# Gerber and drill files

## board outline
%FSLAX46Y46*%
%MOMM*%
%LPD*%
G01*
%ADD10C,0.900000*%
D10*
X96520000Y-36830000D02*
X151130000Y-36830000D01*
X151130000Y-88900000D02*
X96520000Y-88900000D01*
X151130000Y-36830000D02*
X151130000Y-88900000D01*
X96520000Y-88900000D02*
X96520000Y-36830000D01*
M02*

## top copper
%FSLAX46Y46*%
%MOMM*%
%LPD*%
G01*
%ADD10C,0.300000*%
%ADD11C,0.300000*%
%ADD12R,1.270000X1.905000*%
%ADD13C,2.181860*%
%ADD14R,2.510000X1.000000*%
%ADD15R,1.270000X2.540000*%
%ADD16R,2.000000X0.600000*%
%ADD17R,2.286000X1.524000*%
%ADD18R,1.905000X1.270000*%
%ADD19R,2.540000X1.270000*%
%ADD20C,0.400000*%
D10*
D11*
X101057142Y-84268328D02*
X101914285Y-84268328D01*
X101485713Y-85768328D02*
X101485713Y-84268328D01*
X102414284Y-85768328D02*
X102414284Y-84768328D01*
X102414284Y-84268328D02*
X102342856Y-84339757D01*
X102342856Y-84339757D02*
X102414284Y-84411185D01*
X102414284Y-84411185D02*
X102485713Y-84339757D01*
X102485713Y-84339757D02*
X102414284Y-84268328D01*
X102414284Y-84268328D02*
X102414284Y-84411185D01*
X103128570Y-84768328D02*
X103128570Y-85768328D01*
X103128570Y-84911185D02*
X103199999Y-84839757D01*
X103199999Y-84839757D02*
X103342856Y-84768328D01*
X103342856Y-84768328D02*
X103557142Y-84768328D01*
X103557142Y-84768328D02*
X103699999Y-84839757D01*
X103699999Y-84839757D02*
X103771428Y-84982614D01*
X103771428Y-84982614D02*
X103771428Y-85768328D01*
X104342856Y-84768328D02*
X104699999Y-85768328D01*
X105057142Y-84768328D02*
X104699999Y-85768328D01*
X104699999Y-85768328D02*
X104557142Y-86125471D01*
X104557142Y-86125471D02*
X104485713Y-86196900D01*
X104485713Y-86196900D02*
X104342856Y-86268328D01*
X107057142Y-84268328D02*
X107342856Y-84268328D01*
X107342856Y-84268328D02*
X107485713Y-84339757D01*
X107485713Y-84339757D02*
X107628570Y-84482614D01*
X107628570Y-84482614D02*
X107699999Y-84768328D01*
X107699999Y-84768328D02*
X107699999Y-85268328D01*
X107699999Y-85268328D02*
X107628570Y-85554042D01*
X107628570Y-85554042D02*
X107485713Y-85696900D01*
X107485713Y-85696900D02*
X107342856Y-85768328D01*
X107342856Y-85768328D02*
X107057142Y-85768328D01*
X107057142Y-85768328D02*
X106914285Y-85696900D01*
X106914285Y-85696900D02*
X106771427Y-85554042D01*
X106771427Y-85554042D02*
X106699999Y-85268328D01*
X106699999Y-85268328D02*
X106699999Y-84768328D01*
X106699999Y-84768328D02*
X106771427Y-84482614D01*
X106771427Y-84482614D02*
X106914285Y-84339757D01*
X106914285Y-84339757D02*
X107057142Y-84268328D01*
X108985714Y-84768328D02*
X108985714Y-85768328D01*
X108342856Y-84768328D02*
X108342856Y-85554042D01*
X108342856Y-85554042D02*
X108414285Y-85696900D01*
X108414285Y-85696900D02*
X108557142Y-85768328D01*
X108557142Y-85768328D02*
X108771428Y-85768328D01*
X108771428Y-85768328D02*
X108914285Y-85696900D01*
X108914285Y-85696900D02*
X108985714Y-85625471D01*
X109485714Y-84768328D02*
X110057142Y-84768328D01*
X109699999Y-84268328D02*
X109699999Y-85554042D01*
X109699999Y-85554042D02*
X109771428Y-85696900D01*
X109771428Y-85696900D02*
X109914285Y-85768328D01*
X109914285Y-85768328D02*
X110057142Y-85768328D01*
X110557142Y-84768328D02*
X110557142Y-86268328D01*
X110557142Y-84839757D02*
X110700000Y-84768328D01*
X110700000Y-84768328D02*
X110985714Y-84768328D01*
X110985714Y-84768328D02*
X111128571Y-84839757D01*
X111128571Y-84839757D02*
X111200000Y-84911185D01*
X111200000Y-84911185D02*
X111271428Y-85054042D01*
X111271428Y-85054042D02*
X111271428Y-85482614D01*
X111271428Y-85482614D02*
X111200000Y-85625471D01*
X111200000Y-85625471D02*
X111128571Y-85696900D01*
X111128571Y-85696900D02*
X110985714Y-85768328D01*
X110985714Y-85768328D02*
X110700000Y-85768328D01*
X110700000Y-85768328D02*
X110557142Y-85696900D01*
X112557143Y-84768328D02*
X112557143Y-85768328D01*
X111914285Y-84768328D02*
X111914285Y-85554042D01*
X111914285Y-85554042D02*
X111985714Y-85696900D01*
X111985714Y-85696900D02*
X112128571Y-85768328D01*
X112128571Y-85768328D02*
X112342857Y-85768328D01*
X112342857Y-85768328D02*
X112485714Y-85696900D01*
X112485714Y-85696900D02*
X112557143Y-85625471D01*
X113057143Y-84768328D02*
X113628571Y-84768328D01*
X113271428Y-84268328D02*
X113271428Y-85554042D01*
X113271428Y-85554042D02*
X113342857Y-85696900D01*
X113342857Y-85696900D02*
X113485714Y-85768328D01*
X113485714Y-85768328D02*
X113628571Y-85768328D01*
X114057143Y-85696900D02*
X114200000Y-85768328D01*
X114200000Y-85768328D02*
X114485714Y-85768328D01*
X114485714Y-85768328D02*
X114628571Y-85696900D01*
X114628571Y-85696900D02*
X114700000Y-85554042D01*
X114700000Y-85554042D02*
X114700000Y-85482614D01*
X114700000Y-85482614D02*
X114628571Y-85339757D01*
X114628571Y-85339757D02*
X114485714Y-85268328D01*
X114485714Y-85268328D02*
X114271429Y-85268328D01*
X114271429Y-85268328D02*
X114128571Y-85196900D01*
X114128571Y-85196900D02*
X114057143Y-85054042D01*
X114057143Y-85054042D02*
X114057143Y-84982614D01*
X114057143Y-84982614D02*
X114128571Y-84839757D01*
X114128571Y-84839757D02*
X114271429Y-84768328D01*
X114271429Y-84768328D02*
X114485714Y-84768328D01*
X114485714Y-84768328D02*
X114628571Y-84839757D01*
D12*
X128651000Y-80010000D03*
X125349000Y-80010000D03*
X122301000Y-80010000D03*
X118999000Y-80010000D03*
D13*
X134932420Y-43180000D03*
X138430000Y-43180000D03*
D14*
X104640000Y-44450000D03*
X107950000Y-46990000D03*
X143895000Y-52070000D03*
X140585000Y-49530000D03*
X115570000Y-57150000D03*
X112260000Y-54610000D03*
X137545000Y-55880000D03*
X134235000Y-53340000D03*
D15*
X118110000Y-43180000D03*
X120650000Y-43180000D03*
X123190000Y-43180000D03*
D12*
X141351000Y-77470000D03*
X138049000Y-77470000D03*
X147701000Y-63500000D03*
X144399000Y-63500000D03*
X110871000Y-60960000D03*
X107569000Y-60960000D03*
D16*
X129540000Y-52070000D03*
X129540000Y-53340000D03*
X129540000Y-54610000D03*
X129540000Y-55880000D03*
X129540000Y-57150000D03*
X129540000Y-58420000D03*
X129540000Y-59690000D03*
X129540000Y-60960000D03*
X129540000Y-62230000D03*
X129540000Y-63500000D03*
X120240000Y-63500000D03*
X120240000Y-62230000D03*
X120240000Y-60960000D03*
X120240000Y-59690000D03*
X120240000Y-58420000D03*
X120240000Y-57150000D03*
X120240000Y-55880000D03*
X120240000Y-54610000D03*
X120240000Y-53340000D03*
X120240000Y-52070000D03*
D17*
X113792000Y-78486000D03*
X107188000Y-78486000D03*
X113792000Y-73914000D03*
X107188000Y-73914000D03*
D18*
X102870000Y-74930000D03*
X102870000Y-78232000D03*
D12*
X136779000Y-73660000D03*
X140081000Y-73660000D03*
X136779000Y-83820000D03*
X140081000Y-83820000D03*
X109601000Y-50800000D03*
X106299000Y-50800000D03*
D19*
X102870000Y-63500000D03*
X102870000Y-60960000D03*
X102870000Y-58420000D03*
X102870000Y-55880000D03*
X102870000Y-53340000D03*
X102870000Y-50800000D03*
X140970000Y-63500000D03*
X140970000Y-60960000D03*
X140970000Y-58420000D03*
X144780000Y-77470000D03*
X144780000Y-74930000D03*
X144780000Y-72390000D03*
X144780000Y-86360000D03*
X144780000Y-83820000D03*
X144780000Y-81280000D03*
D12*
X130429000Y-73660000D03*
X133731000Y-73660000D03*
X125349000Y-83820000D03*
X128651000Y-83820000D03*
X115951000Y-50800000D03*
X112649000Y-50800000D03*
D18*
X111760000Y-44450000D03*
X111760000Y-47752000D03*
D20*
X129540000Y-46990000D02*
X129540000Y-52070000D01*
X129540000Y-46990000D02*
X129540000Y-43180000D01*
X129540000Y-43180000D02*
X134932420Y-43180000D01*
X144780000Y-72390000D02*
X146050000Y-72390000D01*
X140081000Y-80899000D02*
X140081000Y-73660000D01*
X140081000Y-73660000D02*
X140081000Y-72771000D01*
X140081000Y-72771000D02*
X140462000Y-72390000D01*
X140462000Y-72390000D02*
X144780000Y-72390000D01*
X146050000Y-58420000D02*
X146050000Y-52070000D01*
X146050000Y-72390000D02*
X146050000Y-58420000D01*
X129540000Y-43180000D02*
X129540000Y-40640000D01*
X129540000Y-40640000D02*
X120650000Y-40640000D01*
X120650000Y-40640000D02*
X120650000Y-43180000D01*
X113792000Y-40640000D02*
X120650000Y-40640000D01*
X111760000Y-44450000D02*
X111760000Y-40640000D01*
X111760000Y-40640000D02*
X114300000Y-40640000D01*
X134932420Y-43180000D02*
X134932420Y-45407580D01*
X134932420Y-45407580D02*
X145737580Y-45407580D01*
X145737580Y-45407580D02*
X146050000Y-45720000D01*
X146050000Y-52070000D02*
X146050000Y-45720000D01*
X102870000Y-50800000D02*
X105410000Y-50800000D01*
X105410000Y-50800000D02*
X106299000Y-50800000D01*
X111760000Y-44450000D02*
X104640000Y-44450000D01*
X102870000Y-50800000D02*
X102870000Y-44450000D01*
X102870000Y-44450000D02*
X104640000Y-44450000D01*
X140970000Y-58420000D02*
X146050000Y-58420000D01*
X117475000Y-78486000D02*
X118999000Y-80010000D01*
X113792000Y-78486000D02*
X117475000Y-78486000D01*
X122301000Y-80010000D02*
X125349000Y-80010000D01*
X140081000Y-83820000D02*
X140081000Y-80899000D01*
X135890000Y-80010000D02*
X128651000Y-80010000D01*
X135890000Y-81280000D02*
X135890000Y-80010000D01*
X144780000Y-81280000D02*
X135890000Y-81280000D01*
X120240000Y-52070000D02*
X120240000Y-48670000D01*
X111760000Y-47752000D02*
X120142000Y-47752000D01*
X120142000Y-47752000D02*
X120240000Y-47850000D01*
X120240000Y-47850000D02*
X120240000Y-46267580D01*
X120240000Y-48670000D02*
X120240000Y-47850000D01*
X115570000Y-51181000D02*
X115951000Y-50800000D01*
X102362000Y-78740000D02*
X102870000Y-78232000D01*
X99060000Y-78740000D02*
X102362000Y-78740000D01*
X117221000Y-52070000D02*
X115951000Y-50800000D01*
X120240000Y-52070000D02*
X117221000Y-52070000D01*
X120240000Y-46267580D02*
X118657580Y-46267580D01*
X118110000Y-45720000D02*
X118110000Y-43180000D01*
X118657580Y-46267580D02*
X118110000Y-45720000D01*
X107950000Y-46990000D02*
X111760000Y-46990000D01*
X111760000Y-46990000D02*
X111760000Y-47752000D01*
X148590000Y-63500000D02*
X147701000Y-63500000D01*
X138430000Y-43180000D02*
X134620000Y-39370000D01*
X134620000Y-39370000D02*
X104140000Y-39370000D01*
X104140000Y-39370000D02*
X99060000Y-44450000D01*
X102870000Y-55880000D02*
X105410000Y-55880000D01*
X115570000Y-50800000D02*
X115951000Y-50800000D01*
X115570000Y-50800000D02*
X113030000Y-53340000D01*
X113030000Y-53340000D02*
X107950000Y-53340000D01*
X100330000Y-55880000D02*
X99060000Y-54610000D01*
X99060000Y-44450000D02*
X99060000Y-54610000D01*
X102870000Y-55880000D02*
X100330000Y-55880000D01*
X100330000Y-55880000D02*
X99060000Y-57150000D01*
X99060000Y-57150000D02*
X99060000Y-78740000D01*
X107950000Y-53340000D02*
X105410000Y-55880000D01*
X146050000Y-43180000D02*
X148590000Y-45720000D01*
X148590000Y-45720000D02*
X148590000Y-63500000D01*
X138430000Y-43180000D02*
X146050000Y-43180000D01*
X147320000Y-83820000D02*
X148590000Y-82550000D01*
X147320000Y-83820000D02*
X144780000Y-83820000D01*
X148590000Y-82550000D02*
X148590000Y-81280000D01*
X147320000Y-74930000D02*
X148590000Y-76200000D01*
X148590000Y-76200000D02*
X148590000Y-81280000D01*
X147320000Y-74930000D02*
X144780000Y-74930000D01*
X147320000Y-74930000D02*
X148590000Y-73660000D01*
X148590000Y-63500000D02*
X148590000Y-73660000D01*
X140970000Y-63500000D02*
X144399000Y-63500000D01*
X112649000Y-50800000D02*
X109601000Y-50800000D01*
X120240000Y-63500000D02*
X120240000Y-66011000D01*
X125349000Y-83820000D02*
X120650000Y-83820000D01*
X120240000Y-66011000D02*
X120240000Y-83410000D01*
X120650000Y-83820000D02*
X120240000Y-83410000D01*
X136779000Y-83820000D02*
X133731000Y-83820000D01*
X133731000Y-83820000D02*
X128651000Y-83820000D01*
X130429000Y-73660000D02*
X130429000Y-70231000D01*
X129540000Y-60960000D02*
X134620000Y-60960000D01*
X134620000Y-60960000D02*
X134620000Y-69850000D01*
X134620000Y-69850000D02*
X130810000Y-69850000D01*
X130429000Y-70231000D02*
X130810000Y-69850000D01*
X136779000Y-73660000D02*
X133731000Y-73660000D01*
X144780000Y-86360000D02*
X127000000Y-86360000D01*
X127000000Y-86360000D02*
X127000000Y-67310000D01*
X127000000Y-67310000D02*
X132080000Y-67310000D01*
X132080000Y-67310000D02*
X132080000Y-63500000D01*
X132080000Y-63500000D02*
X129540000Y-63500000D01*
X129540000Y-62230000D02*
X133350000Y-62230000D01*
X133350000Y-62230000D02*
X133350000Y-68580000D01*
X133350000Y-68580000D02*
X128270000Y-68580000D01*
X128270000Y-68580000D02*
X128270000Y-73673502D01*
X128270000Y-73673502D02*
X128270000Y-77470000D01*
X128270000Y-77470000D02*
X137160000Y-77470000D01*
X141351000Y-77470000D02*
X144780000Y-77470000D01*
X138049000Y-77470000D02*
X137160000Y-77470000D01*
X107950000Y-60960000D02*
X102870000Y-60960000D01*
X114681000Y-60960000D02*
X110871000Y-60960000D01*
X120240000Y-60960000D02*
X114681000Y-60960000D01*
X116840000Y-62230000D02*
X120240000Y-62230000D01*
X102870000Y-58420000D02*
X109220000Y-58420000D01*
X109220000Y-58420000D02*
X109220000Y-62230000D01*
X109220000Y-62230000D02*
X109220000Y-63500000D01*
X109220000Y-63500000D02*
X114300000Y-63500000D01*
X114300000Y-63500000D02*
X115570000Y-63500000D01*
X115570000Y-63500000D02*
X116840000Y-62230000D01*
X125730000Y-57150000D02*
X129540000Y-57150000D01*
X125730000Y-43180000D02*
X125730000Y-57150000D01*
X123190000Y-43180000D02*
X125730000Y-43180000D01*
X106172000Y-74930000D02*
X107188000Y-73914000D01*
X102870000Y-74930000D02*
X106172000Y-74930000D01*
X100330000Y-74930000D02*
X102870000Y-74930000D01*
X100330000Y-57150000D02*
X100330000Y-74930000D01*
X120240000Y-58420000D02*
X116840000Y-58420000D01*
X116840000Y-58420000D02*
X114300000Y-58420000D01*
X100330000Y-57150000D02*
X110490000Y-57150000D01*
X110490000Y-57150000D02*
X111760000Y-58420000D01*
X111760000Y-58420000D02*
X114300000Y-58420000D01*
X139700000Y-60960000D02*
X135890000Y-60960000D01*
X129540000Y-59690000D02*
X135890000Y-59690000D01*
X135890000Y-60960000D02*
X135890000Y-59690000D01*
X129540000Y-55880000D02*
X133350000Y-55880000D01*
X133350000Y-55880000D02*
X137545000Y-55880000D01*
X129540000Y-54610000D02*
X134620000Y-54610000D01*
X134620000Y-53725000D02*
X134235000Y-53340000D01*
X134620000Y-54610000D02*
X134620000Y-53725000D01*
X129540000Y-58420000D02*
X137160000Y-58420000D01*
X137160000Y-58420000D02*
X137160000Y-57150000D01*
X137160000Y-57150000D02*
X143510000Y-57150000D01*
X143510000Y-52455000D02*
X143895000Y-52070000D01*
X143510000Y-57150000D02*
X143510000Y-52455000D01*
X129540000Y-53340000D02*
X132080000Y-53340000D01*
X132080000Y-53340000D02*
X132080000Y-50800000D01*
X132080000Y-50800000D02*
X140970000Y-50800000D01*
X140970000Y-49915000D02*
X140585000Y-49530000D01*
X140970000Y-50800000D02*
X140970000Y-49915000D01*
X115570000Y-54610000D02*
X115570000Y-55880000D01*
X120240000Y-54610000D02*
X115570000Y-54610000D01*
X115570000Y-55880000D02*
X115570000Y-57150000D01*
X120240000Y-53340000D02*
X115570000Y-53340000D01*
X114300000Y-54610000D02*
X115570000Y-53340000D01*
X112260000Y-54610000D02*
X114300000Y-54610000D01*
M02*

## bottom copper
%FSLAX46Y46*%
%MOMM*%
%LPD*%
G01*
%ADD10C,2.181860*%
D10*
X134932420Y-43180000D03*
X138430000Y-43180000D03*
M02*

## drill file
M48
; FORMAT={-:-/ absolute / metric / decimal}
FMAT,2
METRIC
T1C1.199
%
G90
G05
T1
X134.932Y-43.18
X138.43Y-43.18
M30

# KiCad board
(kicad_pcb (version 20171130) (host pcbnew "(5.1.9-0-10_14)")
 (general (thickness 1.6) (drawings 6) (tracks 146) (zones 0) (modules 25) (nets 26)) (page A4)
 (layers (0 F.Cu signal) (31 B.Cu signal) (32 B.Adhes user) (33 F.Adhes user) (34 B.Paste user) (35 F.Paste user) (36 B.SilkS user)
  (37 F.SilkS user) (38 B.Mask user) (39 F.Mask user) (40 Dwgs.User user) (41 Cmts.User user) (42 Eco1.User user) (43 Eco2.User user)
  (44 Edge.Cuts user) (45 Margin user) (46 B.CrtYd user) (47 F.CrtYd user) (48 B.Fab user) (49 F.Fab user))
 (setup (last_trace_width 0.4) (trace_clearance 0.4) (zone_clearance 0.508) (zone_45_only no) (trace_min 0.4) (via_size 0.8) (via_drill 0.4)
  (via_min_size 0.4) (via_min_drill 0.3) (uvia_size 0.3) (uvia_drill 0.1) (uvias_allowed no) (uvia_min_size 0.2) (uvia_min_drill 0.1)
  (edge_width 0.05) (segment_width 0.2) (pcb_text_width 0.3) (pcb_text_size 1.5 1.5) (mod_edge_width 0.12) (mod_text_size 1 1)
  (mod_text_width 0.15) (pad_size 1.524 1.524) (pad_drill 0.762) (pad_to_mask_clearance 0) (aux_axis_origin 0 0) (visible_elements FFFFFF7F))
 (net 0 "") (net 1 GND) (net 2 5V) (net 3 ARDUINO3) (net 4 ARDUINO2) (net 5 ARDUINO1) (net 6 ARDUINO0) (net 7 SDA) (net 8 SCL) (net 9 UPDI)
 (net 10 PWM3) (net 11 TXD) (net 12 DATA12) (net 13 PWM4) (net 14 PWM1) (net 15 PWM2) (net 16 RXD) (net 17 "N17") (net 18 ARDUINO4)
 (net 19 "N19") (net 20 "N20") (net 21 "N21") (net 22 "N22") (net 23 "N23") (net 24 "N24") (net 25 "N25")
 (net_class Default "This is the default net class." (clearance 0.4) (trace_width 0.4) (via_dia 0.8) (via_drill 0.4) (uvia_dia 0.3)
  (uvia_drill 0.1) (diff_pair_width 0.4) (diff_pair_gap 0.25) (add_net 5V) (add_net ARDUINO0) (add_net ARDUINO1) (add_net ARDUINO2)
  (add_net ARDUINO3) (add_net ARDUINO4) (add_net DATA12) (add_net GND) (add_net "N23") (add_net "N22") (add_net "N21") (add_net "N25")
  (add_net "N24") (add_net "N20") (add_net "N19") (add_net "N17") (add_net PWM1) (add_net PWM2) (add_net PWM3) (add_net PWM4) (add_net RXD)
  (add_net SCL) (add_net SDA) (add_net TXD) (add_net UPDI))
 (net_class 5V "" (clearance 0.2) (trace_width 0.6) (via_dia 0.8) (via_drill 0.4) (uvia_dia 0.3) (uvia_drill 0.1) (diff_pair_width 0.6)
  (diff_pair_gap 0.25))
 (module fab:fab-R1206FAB (layer F.Cu) (at 127 80.01)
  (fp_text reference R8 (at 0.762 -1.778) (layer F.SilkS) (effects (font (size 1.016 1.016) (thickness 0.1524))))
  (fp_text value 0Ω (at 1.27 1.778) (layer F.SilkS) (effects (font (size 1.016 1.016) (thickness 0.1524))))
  (pad 2 smd rect (at 1.651 0) (size 1.27 1.905) (layers F.Cu F.Paste F.Mask) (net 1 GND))
  (pad 1 smd rect (at -1.651 0) (size 1.27 1.905) (layers F.Cu F.Paste F.Mask) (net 1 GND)))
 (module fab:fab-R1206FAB (layer F.Cu) (at 120.65 80.01)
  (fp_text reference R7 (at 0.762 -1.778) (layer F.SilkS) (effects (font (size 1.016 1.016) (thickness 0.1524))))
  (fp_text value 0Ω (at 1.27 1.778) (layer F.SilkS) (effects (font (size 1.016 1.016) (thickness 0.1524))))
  (pad 2 smd rect (at 1.651 0) (size 1.27 1.905) (layers F.Cu F.Paste F.Mask) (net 1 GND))
  (pad 1 smd rect (at -1.651 0) (size 1.27 1.905) (layers F.Cu F.Paste F.Mask) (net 1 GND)))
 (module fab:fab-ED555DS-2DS (layer F.Cu) (at 136.63168 43.18)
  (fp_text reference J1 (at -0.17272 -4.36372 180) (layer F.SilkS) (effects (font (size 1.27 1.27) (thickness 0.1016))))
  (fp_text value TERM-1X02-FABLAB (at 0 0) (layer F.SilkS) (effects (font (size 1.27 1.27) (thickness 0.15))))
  (pad 2 thru_hole circle (at -1.69926 0) (size 2.18186 2.18186) (drill 1.19888) (layers F&B.Cu F.Paste F.SilkS F.Mask) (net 1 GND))
  (pad 1 thru_hole circle (at 1.79832 0) (size 2.18186 2.18186) (drill 1.19888) (layers F&B.Cu F.Paste F.SilkS F.Mask) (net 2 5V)))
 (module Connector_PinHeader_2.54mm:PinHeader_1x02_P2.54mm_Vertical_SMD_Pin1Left (layer F.Cu) (at 106.295 45.72 180)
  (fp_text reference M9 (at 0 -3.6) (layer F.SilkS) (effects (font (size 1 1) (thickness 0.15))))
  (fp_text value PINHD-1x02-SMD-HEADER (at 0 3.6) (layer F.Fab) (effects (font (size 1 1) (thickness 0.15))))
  (pad 2 smd rect (at 1.655 1.27 180) (size 2.51 1) (layers F.Cu F.Paste F.Mask) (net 1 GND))
  (pad 1 smd rect (at -1.655 -1.27 180) (size 2.51 1) (layers F.Cu F.Paste F.Mask) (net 2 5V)))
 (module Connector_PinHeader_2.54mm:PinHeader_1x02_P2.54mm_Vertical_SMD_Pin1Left (layer F.Cu) (at 142.24 50.8)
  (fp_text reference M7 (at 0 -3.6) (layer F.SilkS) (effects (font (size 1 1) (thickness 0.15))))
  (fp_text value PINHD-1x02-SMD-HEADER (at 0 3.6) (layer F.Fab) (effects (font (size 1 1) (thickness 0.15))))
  (pad 2 smd rect (at 1.655 1.27) (size 2.51 1) (layers F.Cu F.Paste F.Mask) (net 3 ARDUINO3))
  (pad 1 smd rect (at -1.655 -1.27) (size 2.51 1) (layers F.Cu F.Paste F.Mask) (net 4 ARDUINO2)))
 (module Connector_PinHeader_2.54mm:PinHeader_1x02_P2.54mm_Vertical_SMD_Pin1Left (layer F.Cu) (at 113.915 55.88)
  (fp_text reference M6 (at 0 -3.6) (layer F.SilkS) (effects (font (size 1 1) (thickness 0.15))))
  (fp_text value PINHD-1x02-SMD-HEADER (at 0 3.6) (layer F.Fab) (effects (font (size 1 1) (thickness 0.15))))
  (pad 2 smd rect (at 1.655 1.27) (size 2.51 1) (layers F.Cu F.Paste F.Mask) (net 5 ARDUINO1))
  (pad 1 smd rect (at -1.655 -1.27) (size 2.51 1) (layers F.Cu F.Paste F.Mask) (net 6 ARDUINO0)))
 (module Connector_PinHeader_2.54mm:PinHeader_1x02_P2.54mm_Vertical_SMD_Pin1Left (layer F.Cu) (at 135.89 54.61)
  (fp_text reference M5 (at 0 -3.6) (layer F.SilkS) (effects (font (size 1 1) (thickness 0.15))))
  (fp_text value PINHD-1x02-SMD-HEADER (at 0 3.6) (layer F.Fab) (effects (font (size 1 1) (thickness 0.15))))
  (pad 2 smd rect (at 1.655 1.27) (size 2.51 1) (layers F.Cu F.Paste F.Mask) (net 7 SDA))
  (pad 1 smd rect (at -1.655 -1.27) (size 2.51 1) (layers F.Cu F.Paste F.Mask) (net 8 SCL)))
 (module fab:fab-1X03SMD (layer F.Cu) (at 120.65 43.18 270)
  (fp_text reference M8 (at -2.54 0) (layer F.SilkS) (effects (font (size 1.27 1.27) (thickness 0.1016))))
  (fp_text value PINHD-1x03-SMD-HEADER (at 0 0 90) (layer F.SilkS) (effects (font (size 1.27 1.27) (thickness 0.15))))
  (pad 3 smd rect (at 0 2.54 270) (size 2.54 1.27) (layers F.Cu F.Paste F.Mask) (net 2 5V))
  (pad 2 smd rect (at 0 0 270) (size 2.54 1.27) (layers F.Cu F.Paste F.Mask) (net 1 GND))
  (pad 1 smd rect (at 0 -2.54 270) (size 2.54 1.27) (layers F.Cu F.Paste F.Mask) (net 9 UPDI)))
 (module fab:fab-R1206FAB (layer F.Cu) (at 139.7 77.47)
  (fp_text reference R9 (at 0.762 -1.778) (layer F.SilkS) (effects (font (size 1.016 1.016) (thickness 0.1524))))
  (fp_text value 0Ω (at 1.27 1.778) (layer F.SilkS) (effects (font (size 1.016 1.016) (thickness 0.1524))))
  (pad 2 smd rect (at 1.651 0) (size 1.27 1.905) (layers F.Cu F.Paste F.Mask) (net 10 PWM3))
  (pad 1 smd rect (at -1.651 0) (size 1.27 1.905) (layers F.Cu F.Paste F.Mask) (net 10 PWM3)))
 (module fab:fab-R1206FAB (layer F.Cu) (at 146.05 63.5)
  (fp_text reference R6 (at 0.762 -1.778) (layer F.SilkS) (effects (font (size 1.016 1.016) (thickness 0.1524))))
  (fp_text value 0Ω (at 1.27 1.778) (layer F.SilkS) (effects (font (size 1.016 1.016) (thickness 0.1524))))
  (pad 2 smd rect (at 1.651 0) (size 1.27 1.905) (layers F.Cu F.Paste F.Mask) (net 2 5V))
  (pad 1 smd rect (at -1.651 0) (size 1.27 1.905) (layers F.Cu F.Paste F.Mask) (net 2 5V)))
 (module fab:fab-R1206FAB (layer F.Cu) (at 109.22 60.96)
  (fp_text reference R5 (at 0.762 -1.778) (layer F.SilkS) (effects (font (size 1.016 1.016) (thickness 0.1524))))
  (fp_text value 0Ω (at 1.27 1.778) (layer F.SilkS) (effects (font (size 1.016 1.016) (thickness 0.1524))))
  (pad 2 smd rect (at 1.651 0) (size 1.27 1.905) (layers F.Cu F.Paste F.Mask) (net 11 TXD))
  (pad 1 smd rect (at -1.651 0) (size 1.27 1.905) (layers F.Cu F.Paste F.Mask) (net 11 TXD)))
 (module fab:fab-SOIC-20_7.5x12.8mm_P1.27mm (layer F.Cu) (at 124.89 57.785)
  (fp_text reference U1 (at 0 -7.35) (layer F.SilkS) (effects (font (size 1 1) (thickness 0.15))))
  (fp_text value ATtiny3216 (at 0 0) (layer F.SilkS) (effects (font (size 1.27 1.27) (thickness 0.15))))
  (pad 20 smd rect (at 4.65 -5.715) (size 2 0.6) (layers F.Cu) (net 1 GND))
  (pad 19 smd rect (at 4.65 -4.445) (size 2 0.6) (layers F.Cu) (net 4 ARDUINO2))
  (pad 18 smd rect (at 4.65 -3.175) (size 2 0.6) (layers F.Cu) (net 8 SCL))
  (pad 17 smd rect (at 4.65 -1.905) (size 2 0.6) (layers F.Cu) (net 7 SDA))
  (pad 16 smd rect (at 4.65 -0.635) (size 2 0.6) (layers F.Cu) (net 9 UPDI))
  (pad 15 smd rect (at 4.65 0.635) (size 2 0.6) (layers F.Cu) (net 3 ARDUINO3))
  (pad 14 smd rect (at 4.65 1.905) (size 2 0.6) (layers F.Cu) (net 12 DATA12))
  (pad 13 smd rect (at 4.65 3.175) (size 2 0.6) (layers F.Cu) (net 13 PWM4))
  (pad 12 smd rect (at 4.65 4.445) (size 2 0.6) (layers F.Cu) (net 10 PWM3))
  (pad 11 smd rect (at 4.65 5.715) (size 2 0.6) (layers F.Cu) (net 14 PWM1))
  (pad 10 smd rect (at -4.65 5.715) (size 2 0.6) (layers F.Cu) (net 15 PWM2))
  (pad 9 smd rect (at -4.65 4.445) (size 2 0.6) (layers F.Cu) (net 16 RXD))
  (pad 8 smd rect (at -4.65 3.175) (size 2 0.6) (layers F.Cu) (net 11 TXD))
  (pad 7 smd rect (at -4.65 1.905) (size 2 0.6) (layers F.Cu) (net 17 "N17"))
  (pad 6 smd rect (at -4.65 0.635) (size 2 0.6) (layers F.Cu) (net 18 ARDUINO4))
  (pad 5 smd rect (at -4.65 -0.635) (size 2 0.6) (layers F.Cu) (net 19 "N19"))
  (pad 4 smd rect (at -4.65 -1.905) (size 2 0.6) (layers F.Cu) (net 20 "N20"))
  (pad 3 smd rect (at -4.65 -3.175) (size 2 0.6) (layers F.Cu) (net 5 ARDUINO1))
  (pad 2 smd rect (at -4.65 -4.445) (size 2 0.6) (layers F.Cu) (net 6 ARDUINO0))
  (pad 1 smd rect (at -4.65 -5.715) (size 2 0.6) (layers F.Cu) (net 2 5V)))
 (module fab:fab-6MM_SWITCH (layer F.Cu) (at 110.49 76.2)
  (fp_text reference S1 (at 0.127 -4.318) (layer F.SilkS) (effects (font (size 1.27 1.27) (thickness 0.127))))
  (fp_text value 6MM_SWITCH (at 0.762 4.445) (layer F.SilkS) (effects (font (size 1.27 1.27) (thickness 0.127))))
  (pad 4 smd rect (at 3.302 2.286) (size 2.286 1.524) (layers F.Cu F.Paste F.Mask) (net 1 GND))
  (pad 3 smd rect (at -3.302 2.286) (size 2.286 1.524) (layers F.Cu F.Paste F.Mask) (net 1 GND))
  (pad 2 smd rect (at 3.302 -2.286) (size 2.286 1.524) (layers F.Cu F.Paste F.Mask) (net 18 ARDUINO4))
  (pad 1 smd rect (at -3.302 -2.286) (size 2.286 1.524) (layers F.Cu F.Paste F.Mask) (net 18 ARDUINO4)))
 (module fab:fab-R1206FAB (layer F.Cu) (at 102.87 76.581 90)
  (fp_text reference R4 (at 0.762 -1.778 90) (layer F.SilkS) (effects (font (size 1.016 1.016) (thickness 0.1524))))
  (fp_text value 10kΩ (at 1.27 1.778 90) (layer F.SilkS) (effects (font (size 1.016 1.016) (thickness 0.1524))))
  (pad 2 smd rect (at 1.651 0 90) (size 1.27 1.905) (layers F.Cu F.Paste F.Mask) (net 18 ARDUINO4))
  (pad 1 smd rect (at -1.651 0 90) (size 1.27 1.905) (layers F.Cu F.Paste F.Mask) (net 2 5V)))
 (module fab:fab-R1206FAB (layer F.Cu) (at 138.43 73.66 180)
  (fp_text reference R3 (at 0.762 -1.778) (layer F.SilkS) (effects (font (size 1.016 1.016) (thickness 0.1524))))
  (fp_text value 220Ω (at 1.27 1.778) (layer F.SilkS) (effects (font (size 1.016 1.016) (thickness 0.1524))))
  (pad 2 smd rect (at 1.651 0 180) (size 1.27 1.905) (layers F.Cu F.Paste F.Mask) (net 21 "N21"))
  (pad 1 smd rect (at -1.651 0 180) (size 1.27 1.905) (layers F.Cu F.Paste F.Mask) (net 1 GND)))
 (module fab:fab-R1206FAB (layer F.Cu) (at 138.43 83.82 180)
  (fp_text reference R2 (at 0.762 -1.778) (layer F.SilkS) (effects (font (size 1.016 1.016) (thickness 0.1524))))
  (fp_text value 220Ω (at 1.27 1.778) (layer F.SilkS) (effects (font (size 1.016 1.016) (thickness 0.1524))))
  (pad 2 smd rect (at 1.651 0 180) (size 1.27 1.905) (layers F.Cu F.Paste F.Mask) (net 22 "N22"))
  (pad 1 smd rect (at -1.651 0 180) (size 1.27 1.905) (layers F.Cu F.Paste F.Mask) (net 1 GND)))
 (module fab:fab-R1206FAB (layer F.Cu) (at 107.95 50.8)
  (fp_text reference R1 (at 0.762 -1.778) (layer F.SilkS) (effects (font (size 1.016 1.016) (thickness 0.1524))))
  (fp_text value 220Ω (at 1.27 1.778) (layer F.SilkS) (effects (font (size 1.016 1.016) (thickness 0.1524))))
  (pad 2 smd rect (at 1.651 0) (size 1.27 1.905) (layers F.Cu F.Paste F.Mask) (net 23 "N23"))
  (pad 1 smd rect (at -1.651 0) (size 1.27 1.905) (layers F.Cu F.Paste F.Mask) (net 1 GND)))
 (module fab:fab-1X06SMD (layer F.Cu) (at 102.87 57.15)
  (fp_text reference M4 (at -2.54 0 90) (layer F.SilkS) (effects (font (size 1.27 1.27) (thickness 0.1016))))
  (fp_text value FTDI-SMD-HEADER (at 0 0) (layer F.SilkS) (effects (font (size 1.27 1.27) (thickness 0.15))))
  (pad 6 smd rect (at 0 6.35) (size 2.54 1.27) (layers F.Cu F.Paste F.Mask) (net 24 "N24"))
  (pad 5 smd rect (at 0 3.81) (size 2.54 1.27) (layers F.Cu F.Paste F.Mask) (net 11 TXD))
  (pad 4 smd rect (at 0 1.27) (size 2.54 1.27) (layers F.Cu F.Paste F.Mask) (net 16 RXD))
  (pad 3 smd rect (at 0 -1.27) (size 2.54 1.27) (layers F.Cu F.Paste F.Mask) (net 2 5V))
  (pad 2 smd rect (at 0 -3.81) (size 2.54 1.27) (layers F.Cu F.Paste F.Mask) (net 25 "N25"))
  (pad 1 smd rect (at 0 -6.35) (size 2.54 1.27) (layers F.Cu F.Paste F.Mask) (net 1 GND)))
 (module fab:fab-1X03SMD (layer F.Cu) (at 140.97 60.96)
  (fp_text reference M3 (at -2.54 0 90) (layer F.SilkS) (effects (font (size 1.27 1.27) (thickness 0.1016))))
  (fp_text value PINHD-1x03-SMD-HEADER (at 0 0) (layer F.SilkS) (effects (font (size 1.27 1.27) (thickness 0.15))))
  (pad 3 smd rect (at 0 2.54) (size 2.54 1.27) (layers F.Cu F.Paste F.Mask) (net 2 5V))
  (pad 2 smd rect (at 0 0) (size 2.54 1.27) (layers F.Cu F.Paste F.Mask) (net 12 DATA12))
  (pad 1 smd rect (at 0 -2.54) (size 2.54 1.27) (layers F.Cu F.Paste F.Mask) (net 1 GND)))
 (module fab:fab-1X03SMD (layer F.Cu) (at 144.78 74.93)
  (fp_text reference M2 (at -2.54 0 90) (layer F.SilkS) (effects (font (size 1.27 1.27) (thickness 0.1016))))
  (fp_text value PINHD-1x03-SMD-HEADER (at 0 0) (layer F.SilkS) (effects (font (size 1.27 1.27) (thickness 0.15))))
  (pad 3 smd rect (at 0 2.54) (size 2.54 1.27) (layers F.Cu F.Paste F.Mask) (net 10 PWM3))
  (pad 2 smd rect (at 0 0) (size 2.54 1.27) (layers F.Cu F.Paste F.Mask) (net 2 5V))
  (pad 1 smd rect (at 0 -2.54) (size 2.54 1.27) (layers F.Cu F.Paste F.Mask) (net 1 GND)))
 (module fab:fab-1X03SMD (layer F.Cu) (at 144.78 83.82)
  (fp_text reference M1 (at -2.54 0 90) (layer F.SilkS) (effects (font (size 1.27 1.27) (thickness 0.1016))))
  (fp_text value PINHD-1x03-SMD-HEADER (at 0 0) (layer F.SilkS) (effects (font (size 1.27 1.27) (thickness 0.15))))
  (pad 3 smd rect (at 0 2.54) (size 2.54 1.27) (layers F.Cu F.Paste F.Mask) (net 14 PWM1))
  (pad 2 smd rect (at 0 0) (size 2.54 1.27) (layers F.Cu F.Paste F.Mask) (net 2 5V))
  (pad 1 smd rect (at 0 -2.54) (size 2.54 1.27) (layers F.Cu F.Paste F.Mask) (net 1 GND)))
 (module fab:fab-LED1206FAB (layer F.Cu) (at 132.08 73.66 180)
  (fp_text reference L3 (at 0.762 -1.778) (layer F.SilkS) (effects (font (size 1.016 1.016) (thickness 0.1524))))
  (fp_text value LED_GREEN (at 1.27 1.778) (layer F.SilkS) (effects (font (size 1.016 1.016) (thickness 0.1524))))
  (pad 2 smd rect (at 1.651 0 180) (size 1.27 1.905) (layers F.Cu F.Paste F.Mask) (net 13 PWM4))
  (pad 1 smd rect (at -1.651 0 180) (size 1.27 1.905) (layers F.Cu F.Paste F.Mask) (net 21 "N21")))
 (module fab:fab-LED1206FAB (layer F.Cu) (at 127 83.82 180)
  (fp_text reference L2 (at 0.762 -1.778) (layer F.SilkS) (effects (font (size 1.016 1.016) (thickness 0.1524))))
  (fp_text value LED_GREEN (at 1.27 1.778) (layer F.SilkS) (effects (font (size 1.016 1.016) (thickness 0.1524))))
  (pad 2 smd rect (at 1.651 0 180) (size 1.27 1.905) (layers F.Cu F.Paste F.Mask) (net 15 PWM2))
  (pad 1 smd rect (at -1.651 0 180) (size 1.27 1.905) (layers F.Cu F.Paste F.Mask) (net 22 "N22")))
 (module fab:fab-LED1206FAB (layer F.Cu) (at 114.3 50.8)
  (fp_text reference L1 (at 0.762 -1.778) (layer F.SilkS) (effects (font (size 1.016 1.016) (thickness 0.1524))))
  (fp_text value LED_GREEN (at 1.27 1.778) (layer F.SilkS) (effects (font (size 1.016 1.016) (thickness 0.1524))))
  (pad 2 smd rect (at 1.651 0) (size 1.27 1.905) (layers F.Cu F.Paste F.Mask) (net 2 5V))
  (pad 1 smd rect (at -1.651 0) (size 1.27 1.905) (layers F.Cu F.Paste F.Mask) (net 23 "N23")))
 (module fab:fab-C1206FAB (layer F.Cu) (at 111.76 46.101 90)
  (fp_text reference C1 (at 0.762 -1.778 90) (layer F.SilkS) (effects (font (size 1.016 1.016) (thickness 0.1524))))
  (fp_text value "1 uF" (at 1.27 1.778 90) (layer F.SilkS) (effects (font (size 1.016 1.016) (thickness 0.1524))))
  (pad 2 smd rect (at 1.651 0 90) (size 1.27 1.905) (layers F.Cu F.Paste F.Mask) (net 1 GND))
  (pad 1 smd rect (at -1.651 0 90) (size 1.27 1.905) (layers F.Cu F.Paste F.Mask) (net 2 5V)))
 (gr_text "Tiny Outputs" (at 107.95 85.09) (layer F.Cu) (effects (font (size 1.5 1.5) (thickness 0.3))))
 (gr_line (start 96.52 36.83) (end 151.13 36.83) (layer Edge.Cuts) (width 0.9))
 (gr_line (start 151.13 88.9) (end 96.52 88.9) (layer Edge.Cuts) (width 0.9))
 (gr_line (start 151.13 36.83) (end 151.13 88.9) (layer Edge.Cuts) (width 0.9))
 (gr_line (start 96.52 88.9) (end 96.52 36.83) (layer Edge.Cuts) (width 0.9))
 (segment (start 129.54 46.99) (end 129.54 52.07) (width 0.4) (layer F.Cu) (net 1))
 (segment (start 129.54 46.99) (end 129.54 43.18) (width 0.4) (layer F.Cu) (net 1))
 (segment (start 129.54 43.18) (end 134.93242 43.18) (width 0.4) (layer F.Cu) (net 1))
 (segment (start 144.78 72.39) (end 146.05 72.39) (width 0.4) (layer F.Cu) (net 1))
 (segment (start 140.081 80.899) (end 140.081 73.66) (width 0.4) (layer F.Cu) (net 1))
 (segment (start 140.081 73.66) (end 140.081 72.771) (width 0.4) (layer F.Cu) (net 1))
 (segment (start 140.081 72.771) (end 140.462 72.39) (width 0.4) (layer F.Cu) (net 1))
 (segment (start 140.462 72.39) (end 144.78 72.39) (width 0.4) (layer F.Cu) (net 1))
 (segment (start 146.05 58.42) (end 146.05 52.07) (width 0.4) (layer F.Cu) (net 1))
 (segment (start 146.05 72.39) (end 146.05 58.42) (width 0.4) (layer F.Cu) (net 1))
 (segment (start 129.54 43.18) (end 129.54 40.64) (width 0.4) (layer F.Cu) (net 1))
 (segment (start 129.54 40.64) (end 120.65 40.64) (width 0.4) (layer F.Cu) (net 1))
 (segment (start 120.65 40.64) (end 120.65 43.18) (width 0.4) (layer F.Cu) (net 1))
 (segment (start 113.792 40.64) (end 120.65 40.64) (width 0.4) (layer F.Cu) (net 1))
 (segment (start 111.76 44.45) (end 111.76 40.64) (width 0.4) (layer F.Cu) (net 1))
 (segment (start 111.76 40.64) (end 114.3 40.64) (width 0.4) (layer F.Cu) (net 1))
 (segment (start 134.93242 43.18) (end 134.93242 45.40758) (width 0.4) (layer F.Cu) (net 1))
 (segment (start 134.93242 45.40758) (end 145.73758 45.40758) (width 0.4) (layer F.Cu) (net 1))
 (segment (start 145.73758 45.40758) (end 146.05 45.72) (width 0.4) (layer F.Cu) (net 1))
 (segment (start 146.05 52.07) (end 146.05 45.72) (width 0.4) (layer F.Cu) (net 1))
 (segment (start 102.87 50.8) (end 105.41 50.8) (width 0.4) (layer F.Cu) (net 1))
 (segment (start 105.41 50.8) (end 106.299 50.8) (width 0.4) (layer F.Cu) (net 1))
 (segment (start 111.76 44.45) (end 104.64 44.45) (width 0.4) (layer F.Cu) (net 1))
 (segment (start 102.87 50.8) (end 102.87 44.45) (width 0.4) (layer F.Cu) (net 1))
 (segment (start 102.87 44.45) (end 104.64 44.45) (width 0.4) (layer F.Cu) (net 1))
 (segment (start 140.97 58.42) (end 146.05 58.42) (width 0.4) (layer F.Cu) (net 1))
 (segment (start 117.475 78.486) (end 118.999 80.01) (width 0.4) (layer F.Cu) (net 1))
 (segment (start 113.792 78.486) (end 117.475 78.486) (width 0.4) (layer F.Cu) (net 1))
 (segment (start 122.301 80.01) (end 125.349 80.01) (width 0.4) (layer F.Cu) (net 1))
 (segment (start 140.081 83.82) (end 140.081 80.899) (width 0.4) (layer F.Cu) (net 1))
 (segment (start 135.89 80.01) (end 128.651 80.01) (width 0.4) (layer F.Cu) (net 1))
 (segment (start 135.89 81.28) (end 135.89 80.01) (width 0.4) (layer F.Cu) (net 1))
 (segment (start 144.78 81.28) (end 135.89 81.28) (width 0.4) (layer F.Cu) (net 1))
 (segment (start 120.24 52.07) (end 120.24 48.67) (width 0.4) (layer F.Cu) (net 2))
 (segment (start 111.76 47.752) (end 120.142 47.752) (width 0.4) (layer F.Cu) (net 2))
 (segment (start 120.142 47.752) (end 120.24 47.85) (width 0.4) (layer F.Cu) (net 2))
 (segment (start 120.24 47.85) (end 120.24 46.26758) (width 0.4) (layer F.Cu) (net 2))
 (segment (start 120.24 48.67) (end 120.24 47.85) (width 0.4) (layer F.Cu) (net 2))
 (segment (start 115.57 51.181) (end 115.951 50.8) (width 0.4) (layer F.Cu) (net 2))
 (segment (start 102.362 78.74) (end 102.87 78.232) (width 0.4) (layer F.Cu) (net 2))
 (segment (start 99.06 78.74) (end 102.362 78.74) (width 0.4) (layer F.Cu) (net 2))
 (segment (start 117.221 52.07) (end 115.951 50.8) (width 0.4) (layer F.Cu) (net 2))
 (segment (start 120.24 52.07) (end 117.221 52.07) (width 0.4) (layer F.Cu) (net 2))
 (segment (start 120.24 46.26758) (end 118.65758 46.26758) (width 0.4) (layer F.Cu) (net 2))
 (segment (start 118.11 45.72) (end 118.11 43.18) (width 0.4) (layer F.Cu) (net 2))
 (segment (start 118.65758 46.26758) (end 118.11 45.72) (width 0.4) (layer F.Cu) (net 2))
 (segment (start 107.95 46.99) (end 111.76 46.99) (width 0.4) (layer F.Cu) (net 2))
 (segment (start 111.76 46.99) (end 111.76 47.752) (width 0.4) (layer F.Cu) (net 2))
 (segment (start 148.59 63.5) (end 147.701 63.5) (width 0.4) (layer F.Cu) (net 2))
 (segment (start 138.43 43.18) (end 134.62 39.37) (width 0.4) (layer F.Cu) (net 2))
 (segment (start 134.62 39.37) (end 104.14 39.37) (width 0.4) (layer F.Cu) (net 2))
 (segment (start 104.14 39.37) (end 99.06 44.45) (width 0.4) (layer F.Cu) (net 2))
 (segment (start 102.87 55.88) (end 105.41 55.88) (width 0.4) (layer F.Cu) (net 2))
 (segment (start 115.57 50.8) (end 115.951 50.8) (width 0.4) (layer F.Cu) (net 2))
 (segment (start 115.57 50.8) (end 113.03 53.34) (width 0.4) (layer F.Cu) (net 2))
 (segment (start 113.03 53.34) (end 107.95 53.34) (width 0.4) (layer F.Cu) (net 2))
 (segment (start 100.33 55.88) (end 99.06 54.61) (width 0.4) (layer F.Cu) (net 2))
 (segment (start 99.06 44.45) (end 99.06 54.61) (width 0.4) (layer F.Cu) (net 2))
 (segment (start 102.87 55.88) (end 100.33 55.88) (width 0.4) (layer F.Cu) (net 2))
 (segment (start 100.33 55.88) (end 99.06 57.15) (width 0.4) (layer F.Cu) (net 2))
 (segment (start 99.06 57.15) (end 99.06 78.74) (width 0.4) (layer F.Cu) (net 2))
 (segment (start 107.95 53.34) (end 105.41 55.88) (width 0.4) (layer F.Cu) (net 2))
 (segment (start 146.05 43.18) (end 148.59 45.72) (width 0.4) (layer F.Cu) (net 2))
 (segment (start 148.59 45.72) (end 148.59 63.5) (width 0.4) (layer F.Cu) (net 2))
 (segment (start 138.43 43.18) (end 146.05 43.18) (width 0.4) (layer F.Cu) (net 2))
 (segment (start 147.32 83.82) (end 148.59 82.55) (width 0.4) (layer F.Cu) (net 2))
 (segment (start 147.32 83.82) (end 144.78 83.82) (width 0.4) (layer F.Cu) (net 2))
 (segment (start 148.59 82.55) (end 148.59 81.28) (width 0.4) (layer F.Cu) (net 2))
 (segment (start 147.32 74.93) (end 148.59 76.2) (width 0.4) (layer F.Cu) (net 2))
 (segment (start 148.59 76.2) (end 148.59 81.28) (width 0.4) (layer F.Cu) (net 2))
 (segment (start 147.32 74.93) (end 144.78 74.93) (width 0.4) (layer F.Cu) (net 2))
 (segment (start 147.32 74.93) (end 148.59 73.66) (width 0.4) (layer F.Cu) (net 2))
 (segment (start 148.59 63.5) (end 148.59 73.66) (width 0.4) (layer F.Cu) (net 2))
 (segment (start 140.97 63.5) (end 144.399 63.5) (width 0.4) (layer F.Cu) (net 2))
 (segment (start 112.649 50.8) (end 109.601 50.8) (width 0.4) (layer F.Cu) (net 23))
 (segment (start 120.24 63.5) (end 120.24 66.011) (width 0.4) (layer F.Cu) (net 15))
 (segment (start 125.349 83.82) (end 120.65 83.82) (width 0.4) (layer F.Cu) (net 15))
 (segment (start 120.24 66.011) (end 120.24 83.41) (width 0.4) (layer F.Cu) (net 15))
 (segment (start 120.65 83.82) (end 120.24 83.41) (width 0.4) (layer F.Cu) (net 15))
 (segment (start 136.779 83.82) (end 133.731 83.82) (width 0.4) (layer F.Cu) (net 22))
 (segment (start 133.731 83.82) (end 128.651 83.82) (width 0.4) (layer F.Cu) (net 22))
 (segment (start 130.429 73.66) (end 130.429 70.231) (width 0.4) (layer F.Cu) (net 13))
 (segment (start 129.54 60.96) (end 134.62 60.96) (width 0.4) (layer F.Cu) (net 13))
 (segment (start 134.62 60.96) (end 134.62 69.85) (width 0.4) (layer F.Cu) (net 13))
 (segment (start 134.62 69.85) (end 130.81 69.85) (width 0.4) (layer F.Cu) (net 13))
 (segment (start 130.429 70.231) (end 130.81 69.85) (width 0.4) (layer F.Cu) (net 13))
 (segment (start 136.779 73.66) (end 133.731 73.66) (width 0.4) (layer F.Cu) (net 21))
 (segment (start 144.78 86.36) (end 127 86.36) (width 0.4) (layer F.Cu) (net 14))
 (segment (start 127 86.36) (end 127 67.31) (width 0.4) (layer F.Cu) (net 14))
 (segment (start 127 67.31) (end 132.08 67.31) (width 0.4) (layer F.Cu) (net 14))
 (segment (start 132.08 67.31) (end 132.08 63.5) (width 0.4) (layer F.Cu) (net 14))
 (segment (start 132.08 63.5) (end 129.54 63.5) (width 0.4) (layer F.Cu) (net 14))
 (segment (start 129.54 62.23) (end 133.35 62.23) (width 0.4) (layer F.Cu) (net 10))
 (segment (start 133.35 62.23) (end 133.35 68.58) (width 0.4) (layer F.Cu) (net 10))
 (segment (start 133.35 68.58) (end 128.27 68.58) (width 0.4) (layer F.Cu) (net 10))
 (segment (start 128.27 68.58) (end 128.27 73.673502) (width 0.4) (layer F.Cu) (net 10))
 (segment (start 128.27 73.673502) (end 128.27 77.47) (width 0.4) (layer F.Cu) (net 10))
 (segment (start 128.27 77.47) (end 137.16 77.47) (width 0.4) (layer F.Cu) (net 10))
 (segment (start 141.351 77.47) (end 144.78 77.47) (width 0.4) (layer F.Cu) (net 10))
 (segment (start 138.049 77.47) (end 137.16 77.47) (width 0.4) (layer F.Cu) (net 10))
 (segment (start 107.95 60.96) (end 102.87 60.96) (width 0.4) (layer F.Cu) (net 11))
 (segment (start 114.681 60.96) (end 110.871 60.96) (width 0.4) (layer F.Cu) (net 11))
 (segment (start 120.24 60.96) (end 114.681 60.96) (width 0.4) (layer F.Cu) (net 11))
 (segment (start 116.84 62.23) (end 120.24 62.23) (width 0.4) (layer F.Cu) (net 16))
 (segment (start 102.87 58.42) (end 109.22 58.42) (width 0.4) (layer F.Cu) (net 16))
 (segment (start 109.22 58.42) (end 109.22 62.23) (width 0.4) (layer F.Cu) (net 16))
 (segment (start 109.22 62.23) (end 109.22 63.5) (width 0.4) (layer F.Cu) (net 16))
 (segment (start 109.22 63.5) (end 114.3 63.5) (width 0.4) (layer F.Cu) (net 16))
 (segment (start 114.3 63.5) (end 115.57 63.5) (width 0.4) (layer F.Cu) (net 16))
 (segment (start 115.57 63.5) (end 116.84 62.23) (width 0.4) (layer F.Cu) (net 16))
 (segment (start 125.73 57.15) (end 129.54 57.15) (width 0.4) (layer F.Cu) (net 9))
 (segment (start 125.73 43.18) (end 125.73 57.15) (width 0.4) (layer F.Cu) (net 9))
 (segment (start 123.19 43.18) (end 125.73 43.18) (width 0.4) (layer F.Cu) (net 9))
 (segment (start 106.172 74.93) (end 107.188 73.914) (width 0.4) (layer F.Cu) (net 18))
 (segment (start 102.87 74.93) (end 106.172 74.93) (width 0.4) (layer F.Cu) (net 18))
 (segment (start 100.33 74.93) (end 102.87 74.93) (width 0.4) (layer F.Cu) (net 18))
 (segment (start 100.33 57.15) (end 100.33 74.93) (width 0.4) (layer F.Cu) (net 18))
 (segment (start 120.24 58.42) (end 116.84 58.42) (width 0.4) (layer F.Cu) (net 18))
 (segment (start 116.84 58.42) (end 114.3 58.42) (width 0.4) (layer F.Cu) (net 18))
 (segment (start 100.33 57.15) (end 110.49 57.15) (width 0.4) (layer F.Cu) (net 18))
 (segment (start 110.49 57.15) (end 111.76 58.42) (width 0.4) (layer F.Cu) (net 18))
 (segment (start 111.76 58.42) (end 114.3 58.42) (width 0.4) (layer F.Cu) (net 18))
 (segment (start 139.7 60.96) (end 135.89 60.96) (width 0.4) (layer F.Cu) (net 12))
 (segment (start 129.54 59.69) (end 135.89 59.69) (width 0.4) (layer F.Cu) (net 12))
 (segment (start 135.89 60.96) (end 135.89 59.69) (width 0.4) (layer F.Cu) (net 12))
 (segment (start 129.54 55.88) (end 133.35 55.88) (width 0.4) (layer F.Cu) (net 7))
 (segment (start 133.35 55.88) (end 137.545 55.88) (width 0.4) (layer F.Cu) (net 7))
 (segment (start 129.54 54.61) (end 134.62 54.61) (width 0.4) (layer F.Cu) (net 8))
 (segment (start 134.62 53.725) (end 134.235 53.34) (width 0.4) (layer F.Cu) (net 8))
 (segment (start 134.62 54.61) (end 134.62 53.725) (width 0.4) (layer F.Cu) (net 8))
 (segment (start 129.54 58.42) (end 137.16 58.42) (width 0.4) (layer F.Cu) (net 3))
 (segment (start 137.16 58.42) (end 137.16 57.15) (width 0.4) (layer F.Cu) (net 3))
 (segment (start 137.16 57.15) (end 143.51 57.15) (width 0.4) (layer F.Cu) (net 3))
 (segment (start 143.51 52.455) (end 143.895 52.07) (width 0.4) (layer F.Cu) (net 3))
 (segment (start 143.51 57.15) (end 143.51 52.455) (width 0.4) (layer F.Cu) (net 3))
 (segment (start 129.54 53.34) (end 132.08 53.34) (width 0.4) (layer F.Cu) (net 4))
 (segment (start 132.08 53.34) (end 132.08 50.8) (width 0.4) (layer F.Cu) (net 4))
 (segment (start 132.08 50.8) (end 140.97 50.8) (width 0.4) (layer F.Cu) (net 4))
 (segment (start 140.97 49.915) (end 140.585 49.53) (width 0.4) (layer F.Cu) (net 4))
 (segment (start 140.97 50.8) (end 140.97 49.915) (width 0.4) (layer F.Cu) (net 4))
 (segment (start 115.57 54.61) (end 115.57 55.88) (width 0.4) (layer F.Cu) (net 5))
 (segment (start 120.24 54.61) (end 115.57 54.61) (width 0.4) (layer F.Cu) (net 5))
 (segment (start 115.57 55.88) (end 115.57 57.15) (width 0.4) (layer F.Cu) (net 5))
 (segment (start 120.24 53.34) (end 115.57 53.34) (width 0.4) (layer F.Cu) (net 6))
 (segment (start 114.3 54.61) (end 115.57 53.34) (width 0.4) (layer F.Cu) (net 6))
 (segment (start 112.26 54.61) (end 114.3 54.61) (width 0.4) (layer F.Cu) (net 6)))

